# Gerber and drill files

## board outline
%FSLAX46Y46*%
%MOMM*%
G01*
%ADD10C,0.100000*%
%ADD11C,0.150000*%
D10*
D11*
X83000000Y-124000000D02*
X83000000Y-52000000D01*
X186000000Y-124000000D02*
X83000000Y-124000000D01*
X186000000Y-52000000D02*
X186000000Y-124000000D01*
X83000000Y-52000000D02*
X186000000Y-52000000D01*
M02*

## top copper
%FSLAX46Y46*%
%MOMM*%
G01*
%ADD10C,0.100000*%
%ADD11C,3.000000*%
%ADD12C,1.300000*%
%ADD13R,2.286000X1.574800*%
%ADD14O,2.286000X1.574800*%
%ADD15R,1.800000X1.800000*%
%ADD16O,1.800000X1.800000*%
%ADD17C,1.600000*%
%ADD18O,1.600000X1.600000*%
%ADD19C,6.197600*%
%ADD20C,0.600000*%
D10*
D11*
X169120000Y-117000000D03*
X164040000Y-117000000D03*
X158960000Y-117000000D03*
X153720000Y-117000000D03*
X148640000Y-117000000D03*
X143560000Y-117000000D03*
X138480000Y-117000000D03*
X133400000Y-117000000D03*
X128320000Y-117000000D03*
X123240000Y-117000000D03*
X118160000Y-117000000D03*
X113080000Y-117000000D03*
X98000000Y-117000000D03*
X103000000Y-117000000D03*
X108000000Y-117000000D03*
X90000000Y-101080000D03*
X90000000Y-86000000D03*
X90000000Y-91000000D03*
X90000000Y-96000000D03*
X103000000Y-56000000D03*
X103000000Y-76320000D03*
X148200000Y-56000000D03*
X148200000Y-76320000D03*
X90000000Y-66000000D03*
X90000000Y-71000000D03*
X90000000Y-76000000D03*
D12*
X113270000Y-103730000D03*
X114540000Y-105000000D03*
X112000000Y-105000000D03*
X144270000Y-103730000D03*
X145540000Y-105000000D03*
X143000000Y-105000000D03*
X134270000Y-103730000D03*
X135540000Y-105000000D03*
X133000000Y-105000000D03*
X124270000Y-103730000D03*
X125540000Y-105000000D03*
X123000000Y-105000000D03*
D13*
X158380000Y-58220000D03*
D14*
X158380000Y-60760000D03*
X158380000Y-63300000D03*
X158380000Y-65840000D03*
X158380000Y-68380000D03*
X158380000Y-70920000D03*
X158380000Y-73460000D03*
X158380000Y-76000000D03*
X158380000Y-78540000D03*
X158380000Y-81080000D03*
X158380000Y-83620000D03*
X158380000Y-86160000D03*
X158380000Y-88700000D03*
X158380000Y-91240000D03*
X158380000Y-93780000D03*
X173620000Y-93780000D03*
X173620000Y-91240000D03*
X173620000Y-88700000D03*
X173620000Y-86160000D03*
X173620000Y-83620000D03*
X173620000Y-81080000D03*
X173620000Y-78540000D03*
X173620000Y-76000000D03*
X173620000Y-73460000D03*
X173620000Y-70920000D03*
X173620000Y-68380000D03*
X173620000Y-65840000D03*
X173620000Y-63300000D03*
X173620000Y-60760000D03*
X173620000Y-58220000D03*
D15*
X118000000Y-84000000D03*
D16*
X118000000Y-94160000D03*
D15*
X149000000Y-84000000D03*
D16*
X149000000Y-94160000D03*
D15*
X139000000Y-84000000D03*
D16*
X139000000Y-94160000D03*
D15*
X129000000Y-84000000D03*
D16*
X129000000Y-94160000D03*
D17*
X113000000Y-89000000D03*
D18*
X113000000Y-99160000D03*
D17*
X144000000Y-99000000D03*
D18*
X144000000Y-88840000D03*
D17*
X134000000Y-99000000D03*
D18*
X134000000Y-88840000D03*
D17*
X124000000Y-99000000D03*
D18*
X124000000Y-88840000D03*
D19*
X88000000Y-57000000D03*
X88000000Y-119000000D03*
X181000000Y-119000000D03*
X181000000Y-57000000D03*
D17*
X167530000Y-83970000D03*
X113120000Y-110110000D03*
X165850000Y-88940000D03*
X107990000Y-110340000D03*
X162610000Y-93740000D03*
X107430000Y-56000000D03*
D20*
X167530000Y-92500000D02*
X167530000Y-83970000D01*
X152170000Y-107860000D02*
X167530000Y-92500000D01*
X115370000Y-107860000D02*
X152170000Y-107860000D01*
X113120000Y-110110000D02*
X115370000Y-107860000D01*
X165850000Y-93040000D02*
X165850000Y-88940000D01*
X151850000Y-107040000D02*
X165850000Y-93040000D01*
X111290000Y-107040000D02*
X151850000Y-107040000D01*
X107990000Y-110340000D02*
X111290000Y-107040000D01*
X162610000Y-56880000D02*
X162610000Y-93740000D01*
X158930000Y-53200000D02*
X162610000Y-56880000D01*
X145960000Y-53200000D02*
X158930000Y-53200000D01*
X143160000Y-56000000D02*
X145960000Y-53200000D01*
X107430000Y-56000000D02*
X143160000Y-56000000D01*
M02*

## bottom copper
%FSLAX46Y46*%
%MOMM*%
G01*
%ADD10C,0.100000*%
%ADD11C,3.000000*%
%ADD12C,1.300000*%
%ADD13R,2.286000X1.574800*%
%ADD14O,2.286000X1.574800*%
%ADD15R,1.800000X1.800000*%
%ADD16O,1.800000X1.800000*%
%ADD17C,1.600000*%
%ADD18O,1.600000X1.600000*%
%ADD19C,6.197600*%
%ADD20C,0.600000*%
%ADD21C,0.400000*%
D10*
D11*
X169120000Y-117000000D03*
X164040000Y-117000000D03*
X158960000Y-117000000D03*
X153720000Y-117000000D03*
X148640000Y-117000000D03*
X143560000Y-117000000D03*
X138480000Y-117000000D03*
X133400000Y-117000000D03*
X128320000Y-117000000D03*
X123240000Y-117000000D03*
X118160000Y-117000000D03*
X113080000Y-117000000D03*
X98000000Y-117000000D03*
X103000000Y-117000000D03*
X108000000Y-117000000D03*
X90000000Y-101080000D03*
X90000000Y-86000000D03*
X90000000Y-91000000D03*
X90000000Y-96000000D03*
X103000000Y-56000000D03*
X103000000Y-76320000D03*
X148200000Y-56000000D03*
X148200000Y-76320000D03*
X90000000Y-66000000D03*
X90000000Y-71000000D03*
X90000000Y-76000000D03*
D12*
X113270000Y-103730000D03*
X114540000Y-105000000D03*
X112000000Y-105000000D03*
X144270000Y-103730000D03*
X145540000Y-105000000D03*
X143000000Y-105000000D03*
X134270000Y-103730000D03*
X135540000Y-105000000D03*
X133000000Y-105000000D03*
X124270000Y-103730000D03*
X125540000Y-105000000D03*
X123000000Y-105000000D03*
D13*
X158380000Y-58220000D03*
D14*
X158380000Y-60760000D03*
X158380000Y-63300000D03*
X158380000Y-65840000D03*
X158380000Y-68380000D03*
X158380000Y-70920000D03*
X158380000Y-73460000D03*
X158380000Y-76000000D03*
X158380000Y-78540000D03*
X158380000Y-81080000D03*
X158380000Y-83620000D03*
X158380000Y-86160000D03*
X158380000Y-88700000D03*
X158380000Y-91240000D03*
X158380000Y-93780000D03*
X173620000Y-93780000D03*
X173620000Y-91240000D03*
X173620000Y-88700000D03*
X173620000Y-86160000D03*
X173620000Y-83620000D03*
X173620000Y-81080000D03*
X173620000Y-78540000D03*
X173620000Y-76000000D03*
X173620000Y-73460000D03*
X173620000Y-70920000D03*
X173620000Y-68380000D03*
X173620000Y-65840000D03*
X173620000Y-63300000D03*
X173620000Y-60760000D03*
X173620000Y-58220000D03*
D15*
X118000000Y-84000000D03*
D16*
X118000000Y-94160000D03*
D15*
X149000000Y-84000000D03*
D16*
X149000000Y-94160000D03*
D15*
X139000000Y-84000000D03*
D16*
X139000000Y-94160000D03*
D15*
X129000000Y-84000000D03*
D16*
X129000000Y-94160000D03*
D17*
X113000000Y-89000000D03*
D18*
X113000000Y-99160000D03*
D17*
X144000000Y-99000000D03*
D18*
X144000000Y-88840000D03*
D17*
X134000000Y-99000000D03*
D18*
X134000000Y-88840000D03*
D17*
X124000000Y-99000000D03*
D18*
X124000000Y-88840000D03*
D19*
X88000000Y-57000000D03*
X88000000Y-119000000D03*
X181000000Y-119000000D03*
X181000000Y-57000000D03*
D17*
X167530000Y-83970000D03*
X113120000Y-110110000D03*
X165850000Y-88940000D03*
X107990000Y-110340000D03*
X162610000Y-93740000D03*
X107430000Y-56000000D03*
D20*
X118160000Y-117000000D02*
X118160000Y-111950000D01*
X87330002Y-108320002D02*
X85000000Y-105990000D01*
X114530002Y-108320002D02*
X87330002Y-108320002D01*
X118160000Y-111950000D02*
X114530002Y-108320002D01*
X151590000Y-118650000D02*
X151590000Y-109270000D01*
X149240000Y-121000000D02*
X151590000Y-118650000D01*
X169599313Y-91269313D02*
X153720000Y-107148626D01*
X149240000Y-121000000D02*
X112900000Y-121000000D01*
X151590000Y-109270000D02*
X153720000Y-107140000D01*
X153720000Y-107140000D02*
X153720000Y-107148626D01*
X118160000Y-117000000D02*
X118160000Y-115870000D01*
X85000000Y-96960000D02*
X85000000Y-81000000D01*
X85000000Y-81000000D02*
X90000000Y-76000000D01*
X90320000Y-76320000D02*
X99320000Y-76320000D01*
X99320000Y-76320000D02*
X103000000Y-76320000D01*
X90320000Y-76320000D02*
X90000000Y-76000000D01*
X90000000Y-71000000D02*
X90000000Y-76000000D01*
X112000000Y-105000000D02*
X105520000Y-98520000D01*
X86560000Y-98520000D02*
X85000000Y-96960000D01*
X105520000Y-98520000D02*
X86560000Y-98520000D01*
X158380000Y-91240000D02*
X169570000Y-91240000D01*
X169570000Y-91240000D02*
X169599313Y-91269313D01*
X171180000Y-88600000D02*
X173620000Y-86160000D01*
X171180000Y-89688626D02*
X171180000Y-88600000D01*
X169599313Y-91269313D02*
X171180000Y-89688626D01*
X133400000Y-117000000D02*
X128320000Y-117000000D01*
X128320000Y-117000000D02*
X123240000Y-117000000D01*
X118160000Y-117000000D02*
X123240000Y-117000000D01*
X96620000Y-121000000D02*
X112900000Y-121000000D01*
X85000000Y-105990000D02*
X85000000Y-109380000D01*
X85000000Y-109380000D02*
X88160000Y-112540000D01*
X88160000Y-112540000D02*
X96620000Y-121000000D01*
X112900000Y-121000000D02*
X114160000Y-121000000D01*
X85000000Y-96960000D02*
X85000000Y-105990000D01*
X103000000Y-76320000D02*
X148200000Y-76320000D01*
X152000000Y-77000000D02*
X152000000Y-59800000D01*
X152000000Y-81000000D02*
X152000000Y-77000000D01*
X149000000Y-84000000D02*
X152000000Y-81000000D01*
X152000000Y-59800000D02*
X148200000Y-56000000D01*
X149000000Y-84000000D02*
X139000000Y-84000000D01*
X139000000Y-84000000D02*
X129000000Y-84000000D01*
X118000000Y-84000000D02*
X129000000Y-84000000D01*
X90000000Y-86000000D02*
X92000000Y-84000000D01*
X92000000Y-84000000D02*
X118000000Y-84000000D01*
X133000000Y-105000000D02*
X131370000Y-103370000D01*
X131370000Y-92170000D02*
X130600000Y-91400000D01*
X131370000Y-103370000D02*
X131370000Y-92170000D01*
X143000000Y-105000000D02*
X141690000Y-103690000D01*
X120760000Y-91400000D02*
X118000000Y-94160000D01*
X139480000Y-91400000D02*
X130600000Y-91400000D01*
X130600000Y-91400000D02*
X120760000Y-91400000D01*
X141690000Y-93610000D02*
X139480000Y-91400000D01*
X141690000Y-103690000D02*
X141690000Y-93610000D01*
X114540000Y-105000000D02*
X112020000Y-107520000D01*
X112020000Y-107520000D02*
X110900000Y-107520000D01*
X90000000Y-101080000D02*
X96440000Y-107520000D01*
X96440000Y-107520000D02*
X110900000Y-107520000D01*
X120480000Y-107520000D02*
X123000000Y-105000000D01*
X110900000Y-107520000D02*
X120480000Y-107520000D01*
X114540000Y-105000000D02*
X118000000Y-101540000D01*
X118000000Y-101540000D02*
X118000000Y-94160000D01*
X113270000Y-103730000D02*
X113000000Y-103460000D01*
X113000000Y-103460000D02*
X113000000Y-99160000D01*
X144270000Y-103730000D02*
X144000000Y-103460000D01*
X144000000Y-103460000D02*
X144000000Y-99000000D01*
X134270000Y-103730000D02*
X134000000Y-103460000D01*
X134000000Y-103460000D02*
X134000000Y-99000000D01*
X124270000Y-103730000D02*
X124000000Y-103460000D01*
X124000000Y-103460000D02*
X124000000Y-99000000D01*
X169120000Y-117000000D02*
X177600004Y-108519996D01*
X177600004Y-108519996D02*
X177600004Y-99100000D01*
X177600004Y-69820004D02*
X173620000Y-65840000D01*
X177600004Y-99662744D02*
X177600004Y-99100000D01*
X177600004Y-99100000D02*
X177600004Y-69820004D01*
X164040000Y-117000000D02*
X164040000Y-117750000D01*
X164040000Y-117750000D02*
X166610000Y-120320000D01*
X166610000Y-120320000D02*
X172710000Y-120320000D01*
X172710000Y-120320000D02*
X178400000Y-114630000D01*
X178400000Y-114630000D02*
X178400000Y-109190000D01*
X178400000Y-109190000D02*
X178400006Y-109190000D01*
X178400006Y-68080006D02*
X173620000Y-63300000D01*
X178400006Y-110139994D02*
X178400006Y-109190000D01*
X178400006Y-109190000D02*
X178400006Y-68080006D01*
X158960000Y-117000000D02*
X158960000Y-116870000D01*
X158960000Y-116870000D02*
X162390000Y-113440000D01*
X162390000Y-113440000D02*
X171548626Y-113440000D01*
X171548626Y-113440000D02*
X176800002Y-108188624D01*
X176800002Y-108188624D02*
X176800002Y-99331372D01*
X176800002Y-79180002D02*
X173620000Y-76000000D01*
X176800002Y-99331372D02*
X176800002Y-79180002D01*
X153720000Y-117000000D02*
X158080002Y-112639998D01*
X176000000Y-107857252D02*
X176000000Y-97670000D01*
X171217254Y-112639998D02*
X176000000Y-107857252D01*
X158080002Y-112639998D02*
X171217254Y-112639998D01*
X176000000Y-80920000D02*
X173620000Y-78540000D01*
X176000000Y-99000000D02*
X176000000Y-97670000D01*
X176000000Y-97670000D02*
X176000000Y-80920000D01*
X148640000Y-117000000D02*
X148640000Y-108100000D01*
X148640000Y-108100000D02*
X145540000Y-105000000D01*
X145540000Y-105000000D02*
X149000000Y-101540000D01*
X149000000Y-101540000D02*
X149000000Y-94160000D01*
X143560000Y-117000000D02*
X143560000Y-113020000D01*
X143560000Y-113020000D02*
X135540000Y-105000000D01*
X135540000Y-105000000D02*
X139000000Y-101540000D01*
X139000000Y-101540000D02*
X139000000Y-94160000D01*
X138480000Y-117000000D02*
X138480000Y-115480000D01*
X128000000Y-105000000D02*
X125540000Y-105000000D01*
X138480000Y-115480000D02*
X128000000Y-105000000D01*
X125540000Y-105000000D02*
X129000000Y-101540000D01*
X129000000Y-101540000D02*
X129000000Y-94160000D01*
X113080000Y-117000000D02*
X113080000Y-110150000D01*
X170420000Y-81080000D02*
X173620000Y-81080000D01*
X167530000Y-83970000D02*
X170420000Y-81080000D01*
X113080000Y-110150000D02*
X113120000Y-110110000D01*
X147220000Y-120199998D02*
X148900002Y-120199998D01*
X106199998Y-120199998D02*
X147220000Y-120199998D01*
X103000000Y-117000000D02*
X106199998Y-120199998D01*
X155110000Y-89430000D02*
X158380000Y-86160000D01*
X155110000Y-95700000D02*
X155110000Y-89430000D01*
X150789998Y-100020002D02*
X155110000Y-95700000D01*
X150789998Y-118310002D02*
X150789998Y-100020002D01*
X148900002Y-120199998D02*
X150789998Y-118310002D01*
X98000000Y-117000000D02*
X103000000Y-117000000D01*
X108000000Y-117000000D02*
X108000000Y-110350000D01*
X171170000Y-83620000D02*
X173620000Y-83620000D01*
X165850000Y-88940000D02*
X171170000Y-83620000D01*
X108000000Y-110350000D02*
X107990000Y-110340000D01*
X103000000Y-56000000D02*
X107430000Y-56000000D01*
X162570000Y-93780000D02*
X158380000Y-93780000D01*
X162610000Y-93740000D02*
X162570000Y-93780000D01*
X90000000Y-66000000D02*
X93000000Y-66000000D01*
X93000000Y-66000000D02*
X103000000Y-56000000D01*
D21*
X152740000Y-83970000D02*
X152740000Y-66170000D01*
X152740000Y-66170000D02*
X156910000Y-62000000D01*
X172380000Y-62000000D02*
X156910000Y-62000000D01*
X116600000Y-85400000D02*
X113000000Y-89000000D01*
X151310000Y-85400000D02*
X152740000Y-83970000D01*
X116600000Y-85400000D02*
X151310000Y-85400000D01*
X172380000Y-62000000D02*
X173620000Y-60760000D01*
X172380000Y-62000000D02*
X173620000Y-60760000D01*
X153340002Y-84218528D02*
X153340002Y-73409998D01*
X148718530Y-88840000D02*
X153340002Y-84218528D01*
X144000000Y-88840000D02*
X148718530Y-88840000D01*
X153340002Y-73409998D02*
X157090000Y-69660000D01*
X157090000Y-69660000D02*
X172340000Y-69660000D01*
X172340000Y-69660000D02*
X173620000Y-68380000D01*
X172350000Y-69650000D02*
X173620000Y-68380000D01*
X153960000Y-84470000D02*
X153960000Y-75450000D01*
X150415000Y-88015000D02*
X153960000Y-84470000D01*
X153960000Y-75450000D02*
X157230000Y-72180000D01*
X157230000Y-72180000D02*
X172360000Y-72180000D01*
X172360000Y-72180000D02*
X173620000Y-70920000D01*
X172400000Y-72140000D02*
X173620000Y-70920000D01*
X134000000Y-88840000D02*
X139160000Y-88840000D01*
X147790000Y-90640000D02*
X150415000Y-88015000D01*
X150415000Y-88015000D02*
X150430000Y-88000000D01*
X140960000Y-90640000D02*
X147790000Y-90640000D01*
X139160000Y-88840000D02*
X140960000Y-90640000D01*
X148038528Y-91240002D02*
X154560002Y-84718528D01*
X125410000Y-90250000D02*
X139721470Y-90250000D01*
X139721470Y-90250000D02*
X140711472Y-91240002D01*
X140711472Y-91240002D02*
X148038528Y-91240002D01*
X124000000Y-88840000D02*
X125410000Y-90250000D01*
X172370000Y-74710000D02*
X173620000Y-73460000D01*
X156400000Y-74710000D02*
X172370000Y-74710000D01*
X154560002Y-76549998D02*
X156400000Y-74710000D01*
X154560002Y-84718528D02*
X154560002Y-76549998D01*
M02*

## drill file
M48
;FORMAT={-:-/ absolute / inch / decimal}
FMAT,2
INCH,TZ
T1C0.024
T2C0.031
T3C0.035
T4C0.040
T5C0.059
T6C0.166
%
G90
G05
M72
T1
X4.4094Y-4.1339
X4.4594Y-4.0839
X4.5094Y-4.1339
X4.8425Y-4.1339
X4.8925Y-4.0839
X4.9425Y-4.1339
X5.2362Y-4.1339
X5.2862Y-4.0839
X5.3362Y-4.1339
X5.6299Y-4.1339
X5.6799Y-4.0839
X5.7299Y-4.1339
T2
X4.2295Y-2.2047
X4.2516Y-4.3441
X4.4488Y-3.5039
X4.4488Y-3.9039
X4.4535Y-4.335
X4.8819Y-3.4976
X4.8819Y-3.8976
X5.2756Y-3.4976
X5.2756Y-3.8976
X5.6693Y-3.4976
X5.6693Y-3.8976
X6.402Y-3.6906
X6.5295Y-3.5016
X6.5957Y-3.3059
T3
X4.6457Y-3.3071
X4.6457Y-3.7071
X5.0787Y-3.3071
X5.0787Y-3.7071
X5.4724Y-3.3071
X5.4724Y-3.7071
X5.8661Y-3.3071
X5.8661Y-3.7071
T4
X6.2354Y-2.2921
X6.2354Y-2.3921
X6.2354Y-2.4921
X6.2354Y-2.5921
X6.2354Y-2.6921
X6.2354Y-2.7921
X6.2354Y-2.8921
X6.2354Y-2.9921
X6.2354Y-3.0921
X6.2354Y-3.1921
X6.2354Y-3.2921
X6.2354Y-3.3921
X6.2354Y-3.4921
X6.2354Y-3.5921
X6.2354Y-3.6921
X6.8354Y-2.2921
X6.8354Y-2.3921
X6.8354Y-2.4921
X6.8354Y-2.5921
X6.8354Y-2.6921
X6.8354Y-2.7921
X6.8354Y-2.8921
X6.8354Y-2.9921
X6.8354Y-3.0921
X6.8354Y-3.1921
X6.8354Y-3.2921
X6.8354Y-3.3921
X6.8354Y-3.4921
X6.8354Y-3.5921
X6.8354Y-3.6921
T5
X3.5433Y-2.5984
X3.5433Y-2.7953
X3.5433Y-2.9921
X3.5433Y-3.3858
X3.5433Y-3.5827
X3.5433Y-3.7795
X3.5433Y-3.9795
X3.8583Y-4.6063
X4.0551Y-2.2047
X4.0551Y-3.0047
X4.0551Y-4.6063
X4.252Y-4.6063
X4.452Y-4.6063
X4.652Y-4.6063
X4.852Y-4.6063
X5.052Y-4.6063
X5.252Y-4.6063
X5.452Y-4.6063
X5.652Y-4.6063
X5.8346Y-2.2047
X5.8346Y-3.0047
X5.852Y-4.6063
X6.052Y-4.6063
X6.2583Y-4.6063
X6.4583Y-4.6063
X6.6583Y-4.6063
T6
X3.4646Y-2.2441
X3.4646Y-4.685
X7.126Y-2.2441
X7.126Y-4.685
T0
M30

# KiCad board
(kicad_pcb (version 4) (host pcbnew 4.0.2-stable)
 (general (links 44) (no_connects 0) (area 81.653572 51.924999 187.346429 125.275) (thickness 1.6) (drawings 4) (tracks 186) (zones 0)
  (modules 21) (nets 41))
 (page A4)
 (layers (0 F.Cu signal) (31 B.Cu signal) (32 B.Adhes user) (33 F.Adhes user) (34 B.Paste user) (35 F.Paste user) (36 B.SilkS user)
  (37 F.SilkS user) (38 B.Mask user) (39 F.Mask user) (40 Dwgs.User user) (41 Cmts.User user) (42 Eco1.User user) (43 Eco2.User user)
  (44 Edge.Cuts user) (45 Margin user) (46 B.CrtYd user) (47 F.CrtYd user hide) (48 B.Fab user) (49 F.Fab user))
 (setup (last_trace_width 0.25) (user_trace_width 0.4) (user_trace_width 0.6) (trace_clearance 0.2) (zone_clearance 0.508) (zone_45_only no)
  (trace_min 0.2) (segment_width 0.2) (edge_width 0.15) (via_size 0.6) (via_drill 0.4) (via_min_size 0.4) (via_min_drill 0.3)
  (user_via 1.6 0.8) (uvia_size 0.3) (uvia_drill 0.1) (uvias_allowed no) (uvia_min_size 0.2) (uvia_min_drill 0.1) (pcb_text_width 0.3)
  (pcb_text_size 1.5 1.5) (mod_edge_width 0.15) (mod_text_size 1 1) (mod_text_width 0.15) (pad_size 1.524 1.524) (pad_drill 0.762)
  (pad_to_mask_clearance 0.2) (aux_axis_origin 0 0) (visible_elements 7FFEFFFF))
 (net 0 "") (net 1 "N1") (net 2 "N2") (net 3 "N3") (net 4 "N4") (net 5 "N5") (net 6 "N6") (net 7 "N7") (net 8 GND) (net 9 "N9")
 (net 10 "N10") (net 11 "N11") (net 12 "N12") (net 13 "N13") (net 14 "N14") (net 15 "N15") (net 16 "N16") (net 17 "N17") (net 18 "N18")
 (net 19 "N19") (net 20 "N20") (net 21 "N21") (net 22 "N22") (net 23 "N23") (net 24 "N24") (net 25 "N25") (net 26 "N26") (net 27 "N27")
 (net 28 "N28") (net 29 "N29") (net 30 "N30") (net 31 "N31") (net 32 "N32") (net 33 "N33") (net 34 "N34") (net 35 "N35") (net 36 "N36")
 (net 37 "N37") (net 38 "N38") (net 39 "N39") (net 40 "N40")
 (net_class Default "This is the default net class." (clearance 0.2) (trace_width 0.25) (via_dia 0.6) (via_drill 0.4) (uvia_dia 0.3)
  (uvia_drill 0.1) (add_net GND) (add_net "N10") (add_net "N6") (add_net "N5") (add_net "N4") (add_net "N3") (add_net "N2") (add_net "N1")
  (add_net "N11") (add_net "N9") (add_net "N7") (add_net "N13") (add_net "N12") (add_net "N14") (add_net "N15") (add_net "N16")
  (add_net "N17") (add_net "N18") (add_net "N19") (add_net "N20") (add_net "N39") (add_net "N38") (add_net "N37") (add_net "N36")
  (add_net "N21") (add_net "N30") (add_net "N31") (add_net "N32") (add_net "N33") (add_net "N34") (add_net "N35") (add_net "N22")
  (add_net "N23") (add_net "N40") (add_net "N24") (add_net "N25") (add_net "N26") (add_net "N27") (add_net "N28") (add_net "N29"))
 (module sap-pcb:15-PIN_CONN (layer F.Cu) (at 98 117)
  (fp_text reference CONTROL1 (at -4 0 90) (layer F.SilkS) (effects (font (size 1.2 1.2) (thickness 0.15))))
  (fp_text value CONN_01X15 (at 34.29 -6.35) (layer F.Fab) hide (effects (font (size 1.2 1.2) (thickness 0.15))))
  (pad 15 thru_hole circle (at 71.12 0) (size 3 3) (drill 1.5) (layers *.Cu *.Mask F.SilkS) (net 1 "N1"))
  (pad 14 thru_hole circle (at 66.04 0) (size 3 3) (drill 1.5) (layers *.Cu *.Mask F.SilkS) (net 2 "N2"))
  (pad 13 thru_hole circle (at 60.96 0) (size 3 3) (drill 1.5) (layers *.Cu *.Mask F.SilkS) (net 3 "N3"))
  (pad 12 thru_hole circle (at 55.72 0) (size 3 3) (drill 1.5) (layers *.Cu *.Mask F.SilkS) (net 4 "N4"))
  (pad 11 thru_hole circle (at 50.64 0) (size 3 3) (drill 1.5) (layers *.Cu *.Mask F.SilkS) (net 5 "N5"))
  (pad 10 thru_hole circle (at 45.56 0) (size 3 3) (drill 1.5) (layers *.Cu *.Mask F.SilkS) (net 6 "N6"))
  (pad 9 thru_hole circle (at 40.48 0) (size 3 3) (drill 1.5) (layers *.Cu *.Mask F.SilkS) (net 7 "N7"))
  (pad 8 thru_hole circle (at 35.4 0) (size 3 3) (drill 1.5) (layers *.Cu *.Mask F.SilkS) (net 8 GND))
  (pad 7 thru_hole circle (at 30.32 0) (size 3 3) (drill 1.5) (layers *.Cu *.Mask F.SilkS) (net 8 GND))
  (pad 6 thru_hole circle (at 25.24 0) (size 3 3) (drill 1.5) (layers *.Cu *.Mask F.SilkS) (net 8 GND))
  (pad 5 thru_hole circle (at 20.16 0) (size 3 3) (drill 1.5) (layers *.Cu *.Mask F.SilkS) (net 8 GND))
  (pad 4 thru_hole circle (at 15.08 0) (size 3 3) (drill 1.5) (layers *.Cu *.Mask F.SilkS) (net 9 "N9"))
  (pad 1 thru_hole circle (at 0 0) (size 3 3) (drill 1.5) (layers *.Cu *.Mask F.SilkS) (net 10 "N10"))
  (pad 2 thru_hole circle (at 5 0) (size 3 3) (drill 1.5) (layers *.Cu *.Mask F.SilkS) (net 10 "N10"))
  (pad 3 thru_hole circle (at 10 0) (size 3 3) (drill 1.5) (layers *.Cu *.Mask F.SilkS) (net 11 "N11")))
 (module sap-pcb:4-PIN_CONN (layer F.Cu) (at 90 86 270)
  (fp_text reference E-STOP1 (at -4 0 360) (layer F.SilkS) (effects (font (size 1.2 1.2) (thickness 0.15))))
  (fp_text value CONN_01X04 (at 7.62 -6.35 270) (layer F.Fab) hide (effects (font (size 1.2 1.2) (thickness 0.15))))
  (pad 4 thru_hole circle (at 15.08 0 270) (size 3 3) (drill 1.5) (layers *.Cu *.Mask F.SilkS) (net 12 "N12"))
  (pad 1 thru_hole circle (at 0 0 270) (size 3 3) (drill 1.5) (layers *.Cu *.Mask F.SilkS) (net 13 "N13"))
  (pad 2 thru_hole circle (at 5 0 270) (size 3 3) (drill 1.5) (layers *.Cu *.Mask F.SilkS) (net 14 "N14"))
  (pad 3 thru_hole circle (at 10 0 270) (size 3 3) (drill 1.5) (layers *.Cu *.Mask F.SilkS) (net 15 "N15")))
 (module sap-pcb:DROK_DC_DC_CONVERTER (layer F.Cu) (at 103 56)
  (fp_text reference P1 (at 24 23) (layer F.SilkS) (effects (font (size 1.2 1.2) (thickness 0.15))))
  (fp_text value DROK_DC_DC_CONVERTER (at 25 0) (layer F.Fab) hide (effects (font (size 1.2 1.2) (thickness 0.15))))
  (pad 1 thru_hole circle (at 0 0) (size 3 3) (drill 1.5) (layers *.Cu *.Mask F.SilkS) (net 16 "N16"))
  (pad 2 thru_hole circle (at 0 20.32) (size 3 3) (drill 1.5) (layers *.Cu *.Mask F.SilkS) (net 8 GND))
  (pad 3 thru_hole circle (at 45.2 0) (size 3 3) (drill 1.5) (layers *.Cu *.Mask F.SilkS) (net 13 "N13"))
  (pad 4 thru_hole circle (at 45.2 20.32) (size 3 3) (drill 1.5) (layers *.Cu *.Mask F.SilkS) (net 8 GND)))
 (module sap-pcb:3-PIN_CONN (layer F.Cu) (at 90 66 270)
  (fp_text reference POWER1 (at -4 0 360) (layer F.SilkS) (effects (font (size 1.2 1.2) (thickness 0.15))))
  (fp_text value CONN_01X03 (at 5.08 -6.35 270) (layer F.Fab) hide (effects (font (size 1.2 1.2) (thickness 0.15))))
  (pad 1 thru_hole circle (at 0 0 270) (size 3 3) (drill 1.5) (layers *.Cu *.Mask F.SilkS) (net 16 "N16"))
  (pad 2 thru_hole circle (at 5 0 270) (size 3 3) (drill 1.5) (layers *.Cu *.Mask F.SilkS) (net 8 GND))
  (pad 3 thru_hole circle (at 10 0 270) (size 3 3) (drill 1.5) (layers *.Cu *.Mask F.SilkS) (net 8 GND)))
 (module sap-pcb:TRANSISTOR (layer F.Cu) (at 112 105)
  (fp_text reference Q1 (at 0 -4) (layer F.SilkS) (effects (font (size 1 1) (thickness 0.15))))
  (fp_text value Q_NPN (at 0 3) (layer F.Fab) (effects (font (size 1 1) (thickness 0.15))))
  (pad 2 thru_hole circle (at 1.27 -1.27 90) (size 1.3 1.3) (drill 0.6) (layers *.Cu *.Mask F.SilkS) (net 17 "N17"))
  (pad 3 thru_hole circle (at 2.54 0 90) (size 1.3 1.3) (drill 0.6) (layers *.Cu *.Mask F.SilkS) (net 12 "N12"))
  (pad 1 thru_hole circle (at 0 0 90) (size 1.3 1.3) (drill 0.6) (layers *.Cu *.Mask F.SilkS) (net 8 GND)))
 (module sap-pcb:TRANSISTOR (layer F.Cu) (at 143 105)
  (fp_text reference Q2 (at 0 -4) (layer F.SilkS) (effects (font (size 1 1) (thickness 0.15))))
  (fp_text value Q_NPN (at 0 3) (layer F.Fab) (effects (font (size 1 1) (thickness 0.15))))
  (pad 2 thru_hole circle (at 1.27 -1.27 90) (size 1.3 1.3) (drill 0.6) (layers *.Cu *.Mask F.SilkS) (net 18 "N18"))
  (pad 3 thru_hole circle (at 2.54 0 90) (size 1.3 1.3) (drill 0.6) (layers *.Cu *.Mask F.SilkS) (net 5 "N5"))
  (pad 1 thru_hole circle (at 0 0 90) (size 1.3 1.3) (drill 0.6) (layers *.Cu *.Mask F.SilkS) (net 12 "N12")))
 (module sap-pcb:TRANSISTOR (layer F.Cu) (at 133 105)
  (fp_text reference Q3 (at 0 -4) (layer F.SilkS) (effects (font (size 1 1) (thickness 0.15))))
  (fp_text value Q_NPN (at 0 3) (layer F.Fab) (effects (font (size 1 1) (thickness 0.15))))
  (pad 2 thru_hole circle (at 1.27 -1.27 90) (size 1.3 1.3) (drill 0.6) (layers *.Cu *.Mask F.SilkS) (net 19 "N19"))
  (pad 3 thru_hole circle (at 2.54 0 90) (size 1.3 1.3) (drill 0.6) (layers *.Cu *.Mask F.SilkS) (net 6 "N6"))
  (pad 1 thru_hole circle (at 0 0 90) (size 1.3 1.3) (drill 0.6) (layers *.Cu *.Mask F.SilkS) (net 12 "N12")))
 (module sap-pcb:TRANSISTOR (layer F.Cu) (at 123 105)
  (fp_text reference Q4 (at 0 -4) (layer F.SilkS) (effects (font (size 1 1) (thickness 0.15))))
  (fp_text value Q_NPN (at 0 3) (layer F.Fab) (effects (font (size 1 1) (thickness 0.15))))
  (pad 2 thru_hole circle (at 1.27 -1.27 90) (size 1.3 1.3) (drill 0.6) (layers *.Cu *.Mask F.SilkS) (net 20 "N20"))
  (pad 3 thru_hole circle (at 2.54 0 90) (size 1.3 1.3) (drill 0.6) (layers *.Cu *.Mask F.SilkS) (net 7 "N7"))
  (pad 1 thru_hole circle (at 0 0 90) (size 1.3 1.3) (drill 0.6) (layers *.Cu *.Mask F.SilkS) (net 12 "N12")))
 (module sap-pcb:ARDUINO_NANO (layer F.Cu) (at 166 76 270)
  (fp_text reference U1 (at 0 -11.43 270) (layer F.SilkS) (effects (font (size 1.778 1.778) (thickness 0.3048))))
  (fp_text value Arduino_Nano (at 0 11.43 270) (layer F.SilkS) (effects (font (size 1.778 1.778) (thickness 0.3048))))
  (pad 1 thru_hole rect (at -17.78 7.62 270) (size 1.5748 2.286) (drill 1.016) (layers *.Cu *.Mask F.SilkS) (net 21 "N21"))
  (pad 2 thru_hole oval (at -15.24 7.62 270) (size 1.5748 2.286) (drill 1.016) (layers *.Cu *.Mask F.SilkS) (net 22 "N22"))
  (pad 3 thru_hole oval (at -12.7 7.62 270) (size 1.5748 2.286) (drill 1.016) (layers *.Cu *.Mask F.SilkS) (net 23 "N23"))
  (pad 4 thru_hole oval (at -10.16 7.62 270) (size 1.5748 2.286) (drill 1.016) (layers *.Cu *.Mask F.SilkS) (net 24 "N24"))
  (pad 5 thru_hole oval (at -7.62 7.62 270) (size 1.5748 2.286) (drill 1.016) (layers *.Cu *.Mask F.SilkS) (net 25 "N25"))
  (pad 6 thru_hole oval (at -5.08 7.62 270) (size 1.5748 2.286) (drill 1.016) (layers *.Cu *.Mask F.SilkS) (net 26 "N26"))
  (pad 7 thru_hole oval (at -2.54 7.62 270) (size 1.5748 2.286) (drill 1.016) (layers *.Cu *.Mask F.SilkS) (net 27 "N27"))
  (pad 8 thru_hole oval (at 0 7.62 270) (size 1.5748 2.286) (drill 1.016) (layers *.Cu *.Mask F.SilkS) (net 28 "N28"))
  (pad 9 thru_hole oval (at 2.54 7.62 270) (size 1.5748 2.286) (drill 1.016) (layers *.Cu *.Mask F.SilkS) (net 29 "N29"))
  (pad 10 thru_hole oval (at 5.08 7.62 270) (size 1.5748 2.286) (drill 1.016) (layers *.Cu *.Mask F.SilkS) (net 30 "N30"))
  (pad 11 thru_hole oval (at 7.62 7.62 270) (size 1.5748 2.286) (drill 1.016) (layers *.Cu *.Mask F.SilkS) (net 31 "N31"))
  (pad 12 thru_hole oval (at 10.16 7.62 270) (size 1.5748 2.286) (drill 1.016) (layers *.Cu *.Mask F.SilkS) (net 10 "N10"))
  (pad 13 thru_hole oval (at 12.7 7.62 270) (size 1.5748 2.286) (drill 1.016) (layers *.Cu *.Mask F.SilkS) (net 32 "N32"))
  (pad 14 thru_hole oval (at 15.24 7.62 270) (size 1.5748 2.286) (drill 1.016) (layers *.Cu *.Mask F.SilkS) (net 8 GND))
  (pad 15 thru_hole oval (at 17.78 7.62 270) (size 1.5748 2.286) (drill 1.016) (layers *.Cu *.Mask F.SilkS) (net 16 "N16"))
  (pad 16 thru_hole oval (at 17.78 -7.62 270) (size 1.5748 2.286) (drill 1.016) (layers *.Cu *.Mask F.SilkS) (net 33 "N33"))
  (pad 17 thru_hole oval (at 15.24 -7.62 270) (size 1.5748 2.286) (drill 1.016) (layers *.Cu *.Mask F.SilkS) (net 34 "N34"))
  (pad 18 thru_hole oval (at 12.7 -7.62 270) (size 1.5748 2.286) (drill 1.016) (layers *.Cu *.Mask F.SilkS) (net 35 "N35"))
  (pad 19 thru_hole oval (at 10.16 -7.62 270) (size 1.5748 2.286) (drill 1.016) (layers *.Cu *.Mask F.SilkS) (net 8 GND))
  (pad 20 thru_hole oval (at 7.62 -7.62 270) (size 1.5748 2.286) (drill 1.016) (layers *.Cu *.Mask F.SilkS) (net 11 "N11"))
  (pad 21 thru_hole oval (at 5.08 -7.62 270) (size 1.5748 2.286) (drill 1.016) (layers *.Cu *.Mask F.SilkS) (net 9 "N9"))
  (pad 22 thru_hole oval (at 2.54 -7.62 270) (size 1.5748 2.286) (drill 1.016) (layers *.Cu *.Mask F.SilkS) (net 4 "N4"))
  (pad 23 thru_hole oval (at 0 -7.62 270) (size 1.5748 2.286) (drill 1.016) (layers *.Cu *.Mask F.SilkS) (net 3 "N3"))
  (pad 24 thru_hole oval (at -2.54 -7.62 270) (size 1.5748 2.286) (drill 1.016) (layers *.Cu *.Mask F.SilkS) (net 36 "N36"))
  (pad 25 thru_hole oval (at -5.08 -7.62 270) (size 1.5748 2.286) (drill 1.016) (layers *.Cu *.Mask F.SilkS) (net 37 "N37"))
  (pad 26 thru_hole oval (at -7.62 -7.62 270) (size 1.5748 2.286) (drill 1.016) (layers *.Cu *.Mask F.SilkS) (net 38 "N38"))
  (pad 27 thru_hole oval (at -10.16 -7.62 270) (size 1.5748 2.286) (drill 1.016) (layers *.Cu *.Mask F.SilkS) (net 1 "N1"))
  (pad 28 thru_hole oval (at -12.7 -7.62 270) (size 1.5748 2.286) (drill 1.016) (layers *.Cu *.Mask F.SilkS) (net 2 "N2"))
  (pad 29 thru_hole oval (at -15.24 -7.62 270) (size 1.5748 2.286) (drill 1.016) (layers *.Cu *.Mask F.SilkS) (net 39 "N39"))
  (pad 30 thru_hole oval (at -17.78 -7.62 270) (size 1.5748 2.286) (drill 1.016) (layers *.Cu *.Mask F.SilkS) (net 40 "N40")))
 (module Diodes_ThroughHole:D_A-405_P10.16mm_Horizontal (layer F.Cu) (at 118 84 270)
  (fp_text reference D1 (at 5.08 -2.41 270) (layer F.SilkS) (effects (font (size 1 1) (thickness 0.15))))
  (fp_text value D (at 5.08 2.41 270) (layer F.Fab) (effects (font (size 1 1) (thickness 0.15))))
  (pad 1 thru_hole rect (at 0 0 270) (size 1.8 1.8) (drill 0.9) (layers *.Cu *.Mask) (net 13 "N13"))
  (pad 2 thru_hole oval (at 10.16 0 270) (size 1.8 1.8) (drill 0.9) (layers *.Cu *.Mask) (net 12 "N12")))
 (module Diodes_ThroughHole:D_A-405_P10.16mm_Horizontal (layer F.Cu) (at 149 84 270)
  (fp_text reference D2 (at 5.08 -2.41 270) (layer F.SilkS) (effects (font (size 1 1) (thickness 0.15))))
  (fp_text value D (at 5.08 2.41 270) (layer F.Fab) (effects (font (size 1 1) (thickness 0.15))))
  (pad 1 thru_hole rect (at 0 0 270) (size 1.8 1.8) (drill 0.9) (layers *.Cu *.Mask) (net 13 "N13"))
  (pad 2 thru_hole oval (at 10.16 0 270) (size 1.8 1.8) (drill 0.9) (layers *.Cu *.Mask) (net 5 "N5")))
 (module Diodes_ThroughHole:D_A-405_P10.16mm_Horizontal (layer F.Cu) (at 139 84 270)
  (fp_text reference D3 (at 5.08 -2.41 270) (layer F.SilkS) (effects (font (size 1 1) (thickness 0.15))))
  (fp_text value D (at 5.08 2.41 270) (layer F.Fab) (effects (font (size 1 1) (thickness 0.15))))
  (pad 1 thru_hole rect (at 0 0 270) (size 1.8 1.8) (drill 0.9) (layers *.Cu *.Mask) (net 13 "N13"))
  (pad 2 thru_hole oval (at 10.16 0 270) (size 1.8 1.8) (drill 0.9) (layers *.Cu *.Mask) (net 6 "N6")))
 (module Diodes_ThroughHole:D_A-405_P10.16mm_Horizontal (layer F.Cu) (at 129 84 270)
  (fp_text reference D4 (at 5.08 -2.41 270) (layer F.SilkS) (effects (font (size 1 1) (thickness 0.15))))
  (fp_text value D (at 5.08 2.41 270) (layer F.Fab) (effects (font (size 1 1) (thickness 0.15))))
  (pad 1 thru_hole rect (at 0 0 270) (size 1.8 1.8) (drill 0.9) (layers *.Cu *.Mask) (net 13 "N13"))
  (pad 2 thru_hole oval (at 10.16 0 270) (size 1.8 1.8) (drill 0.9) (layers *.Cu *.Mask) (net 7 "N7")))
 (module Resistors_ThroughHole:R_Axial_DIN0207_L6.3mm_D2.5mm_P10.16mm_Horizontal (layer F.Cu) (at 113 89 270)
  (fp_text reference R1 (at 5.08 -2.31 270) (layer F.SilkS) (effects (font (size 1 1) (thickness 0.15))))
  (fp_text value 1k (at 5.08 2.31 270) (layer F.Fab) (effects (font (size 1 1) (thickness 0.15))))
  (pad 1 thru_hole circle (at 0 0 270) (size 1.6 1.6) (drill 0.8) (layers *.Cu *.Mask) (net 39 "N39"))
  (pad 2 thru_hole oval (at 10.16 0 270) (size 1.6 1.6) (drill 0.8) (layers *.Cu *.Mask) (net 17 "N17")))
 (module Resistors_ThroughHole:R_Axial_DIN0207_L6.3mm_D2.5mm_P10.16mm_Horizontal (layer F.Cu) (at 144 99 90)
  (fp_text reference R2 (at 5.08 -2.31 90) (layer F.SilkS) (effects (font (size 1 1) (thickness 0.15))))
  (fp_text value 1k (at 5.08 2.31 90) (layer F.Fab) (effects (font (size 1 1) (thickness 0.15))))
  (pad 1 thru_hole circle (at 0 0 90) (size 1.6 1.6) (drill 0.8) (layers *.Cu *.Mask) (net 18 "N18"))
  (pad 2 thru_hole oval (at 10.16 0 90) (size 1.6 1.6) (drill 0.8) (layers *.Cu *.Mask) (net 38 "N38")))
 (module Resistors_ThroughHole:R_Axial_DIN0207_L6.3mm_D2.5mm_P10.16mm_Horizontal (layer F.Cu) (at 134 99 90)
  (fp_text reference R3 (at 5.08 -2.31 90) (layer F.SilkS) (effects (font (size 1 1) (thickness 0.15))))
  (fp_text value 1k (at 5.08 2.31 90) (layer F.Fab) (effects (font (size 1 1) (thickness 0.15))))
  (pad 1 thru_hole circle (at 0 0 90) (size 1.6 1.6) (drill 0.8) (layers *.Cu *.Mask) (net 19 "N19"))
  (pad 2 thru_hole oval (at 10.16 0 90) (size 1.6 1.6) (drill 0.8) (layers *.Cu *.Mask) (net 37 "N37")))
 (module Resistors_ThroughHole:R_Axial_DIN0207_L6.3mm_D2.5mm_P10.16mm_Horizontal (layer F.Cu) (at 124 99 90)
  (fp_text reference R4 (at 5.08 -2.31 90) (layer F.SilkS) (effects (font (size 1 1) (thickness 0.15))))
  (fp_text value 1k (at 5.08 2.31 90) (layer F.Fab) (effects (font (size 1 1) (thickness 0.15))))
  (pad 1 thru_hole circle (at 0 0 90) (size 1.6 1.6) (drill 0.8) (layers *.Cu *.Mask) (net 20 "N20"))
  (pad 2 thru_hole oval (at 10.16 0 90) (size 1.6 1.6) (drill 0.8) (layers *.Cu *.Mask) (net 36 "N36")))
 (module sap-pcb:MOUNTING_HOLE (layer F.Cu) (at 88 57)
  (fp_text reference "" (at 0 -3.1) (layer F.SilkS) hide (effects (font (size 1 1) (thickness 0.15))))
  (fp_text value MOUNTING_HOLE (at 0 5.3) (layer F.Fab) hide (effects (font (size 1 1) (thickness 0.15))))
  (pad "" np_thru_hole circle (at 0 0) (size 6.1976 6.1976) (drill 4.2164) (layers *.Cu *.Mask)))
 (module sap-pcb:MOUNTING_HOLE (layer F.Cu) (at 88 119)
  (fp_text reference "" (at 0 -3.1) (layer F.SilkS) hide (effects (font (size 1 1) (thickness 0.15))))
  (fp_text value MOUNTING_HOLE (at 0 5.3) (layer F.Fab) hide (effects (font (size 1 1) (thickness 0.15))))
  (pad "" np_thru_hole circle (at 0 0) (size 6.1976 6.1976) (drill 4.2164) (layers *.Cu *.Mask)))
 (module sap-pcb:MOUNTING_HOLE (layer F.Cu) (at 181 119)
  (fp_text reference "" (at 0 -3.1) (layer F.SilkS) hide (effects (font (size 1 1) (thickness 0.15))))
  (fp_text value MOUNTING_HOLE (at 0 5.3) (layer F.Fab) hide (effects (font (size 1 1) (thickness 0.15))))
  (pad "" np_thru_hole circle (at 0 0) (size 6.1976 6.1976) (drill 4.2164) (layers *.Cu *.Mask)))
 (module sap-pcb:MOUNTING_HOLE (layer F.Cu) (at 181 57)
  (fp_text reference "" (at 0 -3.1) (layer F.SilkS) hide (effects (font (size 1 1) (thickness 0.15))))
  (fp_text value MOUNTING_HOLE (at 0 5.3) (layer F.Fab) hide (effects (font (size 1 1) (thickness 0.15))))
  (pad "" np_thru_hole circle (at 0 0) (size 6.1976 6.1976) (drill 4.2164) (layers *.Cu *.Mask)))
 (gr_line (start 83 124) (end 83 52) (angle 90) (layer Edge.Cuts) (width 0.15))
 (gr_line (start 186 124) (end 83 124) (angle 90) (layer Edge.Cuts) (width 0.15))
 (gr_line (start 186 52) (end 186 124) (angle 90) (layer Edge.Cuts) (width 0.15))
 (gr_line (start 83 52) (end 186 52) (angle 90) (layer Edge.Cuts) (width 0.15))
 (segment (start 118.16 117) (end 118.16 111.95) (width 0.6) (layer B.Cu) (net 8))
 (segment (start 87.330002 108.320002) (end 85 105.99) (width 0.6) (layer B.Cu) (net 8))
 (segment (start 114.530002 108.320002) (end 87.330002 108.320002) (width 0.6) (layer B.Cu) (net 8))
 (segment (start 118.16 111.95) (end 114.530002 108.320002) (width 0.6) (layer B.Cu) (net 8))
 (segment (start 151.59 118.65) (end 151.59 109.27) (width 0.6) (layer B.Cu) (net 8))
 (segment (start 149.24 121) (end 151.59 118.65) (width 0.6) (layer B.Cu) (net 8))
 (segment (start 169.599313 91.269313) (end 153.72 107.148626) (width 0.6) (layer B.Cu) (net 8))
 (segment (start 149.24 121) (end 112.9 121) (width 0.6) (layer B.Cu) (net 8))
 (segment (start 151.59 109.27) (end 153.72 107.14) (width 0.6) (layer B.Cu) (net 8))
 (segment (start 153.72 107.14) (end 153.72 107.148626) (width 0.6) (layer B.Cu) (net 8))
 (segment (start 118.16 117) (end 118.16 115.87) (width 0.6) (layer B.Cu) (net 8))
 (segment (start 85 96.96) (end 85 81) (width 0.6) (layer B.Cu) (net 8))
 (segment (start 85 81) (end 90 76) (width 0.6) (layer B.Cu) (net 8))
 (segment (start 90.32 76.32) (end 99.32 76.32) (width 0.6) (layer B.Cu) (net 8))
 (segment (start 99.32 76.32) (end 103 76.32) (width 0.6) (layer B.Cu) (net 8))
 (segment (start 90.32 76.32) (end 90 76) (width 0.6) (layer B.Cu) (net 8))
 (segment (start 90 71) (end 90 76) (width 0.6) (layer B.Cu) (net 8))
 (segment (start 112 105) (end 105.52 98.52) (width 0.6) (layer B.Cu) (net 8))
 (segment (start 86.56 98.52) (end 85 96.96) (width 0.6) (layer B.Cu) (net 8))
 (segment (start 105.52 98.52) (end 86.56 98.52) (width 0.6) (layer B.Cu) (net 8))
 (segment (start 158.38 91.24) (end 169.57 91.24) (width 0.6) (layer B.Cu) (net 8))
 (segment (start 169.57 91.24) (end 169.599313 91.269313) (width 0.6) (layer B.Cu) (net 8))
 (segment (start 171.18 88.6) (end 173.62 86.16) (width 0.6) (layer B.Cu) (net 8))
 (segment (start 171.18 89.688626) (end 171.18 88.6) (width 0.6) (layer B.Cu) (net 8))
 (segment (start 169.599313 91.269313) (end 171.18 89.688626) (width 0.6) (layer B.Cu) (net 8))
 (segment (start 133.4 117) (end 128.32 117) (width 0.6) (layer B.Cu) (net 8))
 (segment (start 128.32 117) (end 123.24 117) (width 0.6) (layer B.Cu) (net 8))
 (segment (start 118.16 117) (end 123.24 117) (width 0.6) (layer B.Cu) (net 8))
 (segment (start 96.62 121) (end 112.9 121) (width 0.6) (layer B.Cu) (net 8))
 (segment (start 85 105.99) (end 85 109.38) (width 0.6) (layer B.Cu) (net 8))
 (segment (start 85 109.38) (end 88.16 112.54) (width 0.6) (layer B.Cu) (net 8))
 (segment (start 88.16 112.54) (end 96.62 121) (width 0.6) (layer B.Cu) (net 8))
 (segment (start 112.9 121) (end 114.16 121) (width 0.6) (layer B.Cu) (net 8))
 (segment (start 85 96.96) (end 85 105.99) (width 0.6) (layer B.Cu) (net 8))
 (segment (start 103 76.32) (end 148.2 76.32) (width 0.6) (layer B.Cu) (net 8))
 (segment (start 152 77) (end 152 59.8) (width 0.6) (layer B.Cu) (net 13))
 (segment (start 152 81) (end 152 77) (width 0.6) (layer B.Cu) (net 13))
 (segment (start 149 84) (end 152 81) (width 0.6) (layer B.Cu) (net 13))
 (segment (start 152 59.8) (end 148.2 56) (width 0.6) (layer B.Cu) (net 13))
 (segment (start 149 84) (end 139 84) (width 0.6) (layer B.Cu) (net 13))
 (segment (start 139 84) (end 129 84) (width 0.6) (layer B.Cu) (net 13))
 (segment (start 118 84) (end 129 84) (width 0.6) (layer B.Cu) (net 13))
 (segment (start 90 86) (end 92 84) (width 0.6) (layer B.Cu) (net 13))
 (segment (start 92 84) (end 118 84) (width 0.6) (layer B.Cu) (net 13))
 (segment (start 133 105) (end 131.37 103.37) (width 0.6) (layer B.Cu) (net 12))
 (segment (start 131.37 92.17) (end 130.6 91.4) (width 0.6) (layer B.Cu) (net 12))
 (segment (start 131.37 103.37) (end 131.37 92.17) (width 0.6) (layer B.Cu) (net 12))
 (segment (start 143 105) (end 141.69 103.69) (width 0.6) (layer B.Cu) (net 12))
 (segment (start 120.76 91.4) (end 118 94.16) (width 0.6) (layer B.Cu) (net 12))
 (segment (start 139.48 91.4) (end 130.6 91.4) (width 0.6) (layer B.Cu) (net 12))
 (segment (start 130.6 91.4) (end 120.76 91.4) (width 0.6) (layer B.Cu) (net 12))
 (segment (start 141.69 93.61) (end 139.48 91.4) (width 0.6) (layer B.Cu) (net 12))
 (segment (start 141.69 103.69) (end 141.69 93.61) (width 0.6) (layer B.Cu) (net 12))
 (segment (start 114.54 105) (end 112.02 107.52) (width 0.6) (layer B.Cu) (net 12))
 (segment (start 112.02 107.52) (end 110.9 107.52) (width 0.6) (layer B.Cu) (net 12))
 (segment (start 90 101.08) (end 96.44 107.52) (width 0.6) (layer B.Cu) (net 12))
 (segment (start 96.44 107.52) (end 110.9 107.52) (width 0.6) (layer B.Cu) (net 12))
 (segment (start 120.48 107.52) (end 123 105) (width 0.6) (layer B.Cu) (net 12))
 (segment (start 110.9 107.52) (end 120.48 107.52) (width 0.6) (layer B.Cu) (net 12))
 (segment (start 114.54 105) (end 118 101.54) (width 0.6) (layer B.Cu) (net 12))
 (segment (start 118 101.54) (end 118 94.16) (width 0.6) (layer B.Cu) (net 12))
 (segment (start 113.27 103.73) (end 113 103.46) (width 0.6) (layer B.Cu) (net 17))
 (segment (start 113 103.46) (end 113 99.16) (width 0.6) (layer B.Cu) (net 17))
 (segment (start 144.27 103.73) (end 144 103.46) (width 0.6) (layer B.Cu) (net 18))
 (segment (start 144 103.46) (end 144 99) (width 0.6) (layer B.Cu) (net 18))
 (segment (start 134.27 103.73) (end 134 103.46) (width 0.6) (layer B.Cu) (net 19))
 (segment (start 134 103.46) (end 134 99) (width 0.6) (layer B.Cu) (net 19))
 (segment (start 124.27 103.73) (end 124 103.46) (width 0.6) (layer B.Cu) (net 20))
 (segment (start 124 103.46) (end 124 99) (width 0.6) (layer B.Cu) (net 20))
 (segment (start 169.12 117) (end 177.600004 108.519996) (width 0.6) (layer B.Cu) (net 1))
 (segment (start 177.600004 108.519996) (end 177.600004 99.1) (width 0.6) (layer B.Cu) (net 1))
 (segment (start 177.600004 69.820004) (end 173.62 65.84) (width 0.6) (layer B.Cu) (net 1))
 (segment (start 177.600004 99.662744) (end 177.600004 99.1) (width 0.6) (layer B.Cu) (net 1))
 (segment (start 177.600004 99.1) (end 177.600004 69.820004) (width 0.6) (layer B.Cu) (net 1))
 (segment (start 164.04 117) (end 164.04 117.75) (width 0.6) (layer B.Cu) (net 2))
 (segment (start 164.04 117.75) (end 166.61 120.32) (width 0.6) (layer B.Cu) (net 2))
 (segment (start 166.61 120.32) (end 172.71 120.32) (width 0.6) (layer B.Cu) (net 2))
 (segment (start 172.71 120.32) (end 178.4 114.63) (width 0.6) (layer B.Cu) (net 2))
 (segment (start 178.4 114.63) (end 178.4 109.19) (width 0.6) (layer B.Cu) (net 2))
 (segment (start 178.4 109.19) (end 178.400006 109.19) (width 0.6) (layer B.Cu) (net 2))
 (segment (start 178.400006 68.080006) (end 173.62 63.3) (width 0.6) (layer B.Cu) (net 2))
 (segment (start 178.400006 110.139994) (end 178.400006 109.19) (width 0.6) (layer B.Cu) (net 2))
 (segment (start 178.400006 109.19) (end 178.400006 68.080006) (width 0.6) (layer B.Cu) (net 2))
 (segment (start 158.96 117) (end 158.96 116.87) (width 0.6) (layer B.Cu) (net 3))
 (segment (start 158.96 116.87) (end 162.39 113.44) (width 0.6) (layer B.Cu) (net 3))
 (segment (start 162.39 113.44) (end 171.548626 113.44) (width 0.6) (layer B.Cu) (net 3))
 (segment (start 171.548626 113.44) (end 176.800002 108.188624) (width 0.6) (layer B.Cu) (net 3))
 (segment (start 176.800002 108.188624) (end 176.800002 99.331372) (width 0.6) (layer B.Cu) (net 3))
 (segment (start 176.800002 79.180002) (end 173.62 76) (width 0.6) (layer B.Cu) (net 3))
 (segment (start 176.800002 99.331372) (end 176.800002 79.180002) (width 0.6) (layer B.Cu) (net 3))
 (segment (start 153.72 117) (end 158.080002 112.639998) (width 0.6) (layer B.Cu) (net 4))
 (segment (start 176 107.857252) (end 176 97.67) (width 0.6) (layer B.Cu) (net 4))
 (segment (start 171.217254 112.639998) (end 176 107.857252) (width 0.6) (layer B.Cu) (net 4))
 (segment (start 158.080002 112.639998) (end 171.217254 112.639998) (width 0.6) (layer B.Cu) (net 4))
 (segment (start 176 80.92) (end 173.62 78.54) (width 0.6) (layer B.Cu) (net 4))
 (segment (start 176 99) (end 176 97.67) (width 0.6) (layer B.Cu) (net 4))
 (segment (start 176 97.67) (end 176 80.92) (width 0.6) (layer B.Cu) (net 4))
 (segment (start 148.64 117) (end 148.64 108.1) (width 0.6) (layer B.Cu) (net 5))
 (segment (start 148.64 108.1) (end 145.54 105) (width 0.6) (layer B.Cu) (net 5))
 (segment (start 145.54 105) (end 149 101.54) (width 0.6) (layer B.Cu) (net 5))
 (segment (start 149 101.54) (end 149 94.16) (width 0.6) (layer B.Cu) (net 5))
 (segment (start 143.56 117) (end 143.56 113.02) (width 0.6) (layer B.Cu) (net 6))
 (segment (start 143.56 113.02) (end 135.54 105) (width 0.6) (layer B.Cu) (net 6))
 (segment (start 135.54 105) (end 139 101.54) (width 0.6) (layer B.Cu) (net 6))
 (segment (start 139 101.54) (end 139 94.16) (width 0.6) (layer B.Cu) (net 6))
 (segment (start 138.48 117) (end 138.48 115.48) (width 0.6) (layer B.Cu) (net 7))
 (segment (start 128 105) (end 125.54 105) (width 0.6) (layer B.Cu) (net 7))
 (segment (start 138.48 115.48) (end 128 105) (width 0.6) (layer B.Cu) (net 7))
 (segment (start 125.54 105) (end 129 101.54) (width 0.6) (layer B.Cu) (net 7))
 (segment (start 129 101.54) (end 129 94.16) (width 0.6) (layer B.Cu) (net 7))
 (segment (start 113.08 117) (end 113.08 110.15) (width 0.6) (layer B.Cu) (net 9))
 (segment (start 170.42 81.08) (end 173.62 81.08) (width 0.6) (layer B.Cu) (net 9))
 (segment (start 167.53 83.97) (end 170.42 81.08) (width 0.6) (layer B.Cu) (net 9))
 (via (at 167.53 83.97) (size 1.6) (drill 0.8) (layers F.Cu B.Cu) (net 9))
 (segment (start 167.53 92.5) (end 167.53 83.97) (width 0.6) (layer F.Cu) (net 9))
 (segment (start 152.17 107.86) (end 167.53 92.5) (width 0.6) (layer F.Cu) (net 9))
 (segment (start 115.37 107.86) (end 152.17 107.86) (width 0.6) (layer F.Cu) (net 9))
 (segment (start 113.12 110.11) (end 115.37 107.86) (width 0.6) (layer F.Cu) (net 9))
 (via (at 113.12 110.11) (size 1.6) (drill 0.8) (layers F.Cu B.Cu) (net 9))
 (segment (start 113.08 110.15) (end 113.12 110.11) (width 0.6) (layer B.Cu) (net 9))
 (segment (start 147.22 120.199998) (end 148.900002 120.199998) (width 0.6) (layer B.Cu) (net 10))
 (segment (start 106.199998 120.199998) (end 147.22 120.199998) (width 0.6) (layer B.Cu) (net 10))
 (segment (start 103 117) (end 106.199998 120.199998) (width 0.6) (layer B.Cu) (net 10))
 (segment (start 155.11 89.43) (end 158.38 86.16) (width 0.6) (layer B.Cu) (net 10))
 (segment (start 155.11 95.7) (end 155.11 89.43) (width 0.6) (layer B.Cu) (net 10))
 (segment (start 150.789998 100.020002) (end 155.11 95.7) (width 0.6) (layer B.Cu) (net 10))
 (segment (start 150.789998 118.310002) (end 150.789998 100.020002) (width 0.6) (layer B.Cu) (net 10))
 (segment (start 148.900002 120.199998) (end 150.789998 118.310002) (width 0.6) (layer B.Cu) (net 10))
 (segment (start 98 117) (end 103 117) (width 0.6) (layer B.Cu) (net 10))
 (segment (start 108 117) (end 108 110.35) (width 0.6) (layer B.Cu) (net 11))
 (segment (start 171.17 83.62) (end 173.62 83.62) (width 0.6) (layer B.Cu) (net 11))
 (segment (start 165.85 88.94) (end 171.17 83.62) (width 0.6) (layer B.Cu) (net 11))
 (via (at 165.85 88.94) (size 1.6) (drill 0.8) (layers F.Cu B.Cu) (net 11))
 (segment (start 165.85 93.04) (end 165.85 88.94) (width 0.6) (layer F.Cu) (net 11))
 (segment (start 151.85 107.04) (end 165.85 93.04) (width 0.6) (layer F.Cu) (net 11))
 (segment (start 111.29 107.04) (end 151.85 107.04) (width 0.6) (layer F.Cu) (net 11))
 (segment (start 107.99 110.34) (end 111.29 107.04) (width 0.6) (layer F.Cu) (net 11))
 (via (at 107.99 110.34) (size 1.6) (drill 0.8) (layers F.Cu B.Cu) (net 11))
 (segment (start 108 110.35) (end 107.99 110.34) (width 0.6) (layer B.Cu) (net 11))
 (segment (start 103 56) (end 107.43 56) (width 0.6) (layer B.Cu) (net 16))
 (segment (start 162.57 93.78) (end 158.38 93.78) (width 0.6) (layer B.Cu) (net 16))
 (segment (start 162.61 93.74) (end 162.57 93.78) (width 0.6) (layer B.Cu) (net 16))
 (via (at 162.61 93.74) (size 1.6) (drill 0.8) (layers F.Cu B.Cu) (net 16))
 (segment (start 162.61 56.88) (end 162.61 93.74) (width 0.6) (layer F.Cu) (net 16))
 (segment (start 158.93 53.2) (end 162.61 56.88) (width 0.6) (layer F.Cu) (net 16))
 (segment (start 145.96 53.2) (end 158.93 53.2) (width 0.6) (layer F.Cu) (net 16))
 (segment (start 143.16 56) (end 145.96 53.2) (width 0.6) (layer F.Cu) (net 16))
 (segment (start 107.43 56) (end 143.16 56) (width 0.6) (layer F.Cu) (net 16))
 (via (at 107.43 56) (size 1.6) (drill 0.8) (layers F.Cu B.Cu) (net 16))
 (segment (start 90 66) (end 93 66) (width 0.6) (layer B.Cu) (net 16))
 (segment (start 93 66) (end 103 56) (width 0.6) (layer B.Cu) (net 16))
 (segment (start 152.74 83.97) (end 152.74 66.17) (width 0.4) (layer B.Cu) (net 39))
 (segment (start 152.74 66.17) (end 156.91 62) (width 0.4) (layer B.Cu) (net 39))
 (segment (start 172.38 62) (end 156.91 62) (width 0.4) (layer B.Cu) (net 39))
 (segment (start 116.6 85.4) (end 113 89) (width 0.4) (layer B.Cu) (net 39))
 (segment (start 151.31 85.4) (end 152.74 83.97) (width 0.4) (layer B.Cu) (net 39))
 (segment (start 116.6 85.4) (end 151.31 85.4) (width 0.4) (layer B.Cu) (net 39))
 (segment (start 172.38 62) (end 173.62 60.76) (width 0.4) (layer B.Cu) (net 39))
 (segment (start 172.38 62) (end 173.62 60.76) (width 0.4) (layer B.Cu) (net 39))
 (segment (start 153.340002 84.218528) (end 153.340002 73.409998) (width 0.4) (layer B.Cu) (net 38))
 (segment (start 148.71853 88.84) (end 153.340002 84.218528) (width 0.4) (layer B.Cu) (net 38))
 (segment (start 144 88.84) (end 148.71853 88.84) (width 0.4) (layer B.Cu) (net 38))
 (segment (start 153.340002 73.409998) (end 157.09 69.66) (width 0.4) (layer B.Cu) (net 38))
 (segment (start 157.09 69.66) (end 172.34 69.66) (width 0.4) (layer B.Cu) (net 38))
 (segment (start 172.34 69.66) (end 173.62 68.38) (width 0.4) (layer B.Cu) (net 38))
 (segment (start 172.35 69.65) (end 173.62 68.38) (width 0.4) (layer B.Cu) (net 38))
 (segment (start 153.96 84.47) (end 153.96 75.45) (width 0.4) (layer B.Cu) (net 37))
 (segment (start 150.415 88.015) (end 153.96 84.47) (width 0.4) (layer B.Cu) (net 37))
 (segment (start 153.96 75.45) (end 157.23 72.18) (width 0.4) (layer B.Cu) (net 37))
 (segment (start 157.23 72.18) (end 172.36 72.18) (width 0.4) (layer B.Cu) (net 37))
 (segment (start 172.36 72.18) (end 173.62 70.92) (width 0.4) (layer B.Cu) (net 37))
 (segment (start 172.4 72.14) (end 173.62 70.92) (width 0.4) (layer B.Cu) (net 37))
 (segment (start 134 88.84) (end 139.16 88.84) (width 0.4) (layer B.Cu) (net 37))
 (segment (start 147.79 90.64) (end 150.415 88.015) (width 0.4) (layer B.Cu) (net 37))
 (segment (start 150.415 88.015) (end 150.43 88) (width 0.4) (layer B.Cu) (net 37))
 (segment (start 140.96 90.64) (end 147.79 90.64) (width 0.4) (layer B.Cu) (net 37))
 (segment (start 139.16 88.84) (end 140.96 90.64) (width 0.4) (layer B.Cu) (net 37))
 (segment (start 148.038528 91.240002) (end 154.560002 84.718528) (width 0.4) (layer B.Cu) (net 36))
 (segment (start 125.41 90.25) (end 139.72147 90.25) (width 0.4) (layer B.Cu) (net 36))
 (segment (start 139.72147 90.25) (end 140.711472 91.240002) (width 0.4) (layer B.Cu) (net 36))
 (segment (start 140.711472 91.240002) (end 148.038528 91.240002) (width 0.4) (layer B.Cu) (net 36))
 (segment (start 124 88.84) (end 125.41 90.25) (width 0.4) (layer B.Cu) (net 36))
 (segment (start 172.37 74.71) (end 173.62 73.46) (width 0.4) (layer B.Cu) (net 36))
 (segment (start 156.4 74.71) (end 172.37 74.71) (width 0.4) (layer B.Cu) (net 36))
 (segment (start 154.560002 76.549998) (end 156.4 74.71) (width 0.4) (layer B.Cu) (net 36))
 (segment (start 154.560002 84.718528) (end 154.560002 76.549998) (width 0.4) (layer B.Cu) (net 36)))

